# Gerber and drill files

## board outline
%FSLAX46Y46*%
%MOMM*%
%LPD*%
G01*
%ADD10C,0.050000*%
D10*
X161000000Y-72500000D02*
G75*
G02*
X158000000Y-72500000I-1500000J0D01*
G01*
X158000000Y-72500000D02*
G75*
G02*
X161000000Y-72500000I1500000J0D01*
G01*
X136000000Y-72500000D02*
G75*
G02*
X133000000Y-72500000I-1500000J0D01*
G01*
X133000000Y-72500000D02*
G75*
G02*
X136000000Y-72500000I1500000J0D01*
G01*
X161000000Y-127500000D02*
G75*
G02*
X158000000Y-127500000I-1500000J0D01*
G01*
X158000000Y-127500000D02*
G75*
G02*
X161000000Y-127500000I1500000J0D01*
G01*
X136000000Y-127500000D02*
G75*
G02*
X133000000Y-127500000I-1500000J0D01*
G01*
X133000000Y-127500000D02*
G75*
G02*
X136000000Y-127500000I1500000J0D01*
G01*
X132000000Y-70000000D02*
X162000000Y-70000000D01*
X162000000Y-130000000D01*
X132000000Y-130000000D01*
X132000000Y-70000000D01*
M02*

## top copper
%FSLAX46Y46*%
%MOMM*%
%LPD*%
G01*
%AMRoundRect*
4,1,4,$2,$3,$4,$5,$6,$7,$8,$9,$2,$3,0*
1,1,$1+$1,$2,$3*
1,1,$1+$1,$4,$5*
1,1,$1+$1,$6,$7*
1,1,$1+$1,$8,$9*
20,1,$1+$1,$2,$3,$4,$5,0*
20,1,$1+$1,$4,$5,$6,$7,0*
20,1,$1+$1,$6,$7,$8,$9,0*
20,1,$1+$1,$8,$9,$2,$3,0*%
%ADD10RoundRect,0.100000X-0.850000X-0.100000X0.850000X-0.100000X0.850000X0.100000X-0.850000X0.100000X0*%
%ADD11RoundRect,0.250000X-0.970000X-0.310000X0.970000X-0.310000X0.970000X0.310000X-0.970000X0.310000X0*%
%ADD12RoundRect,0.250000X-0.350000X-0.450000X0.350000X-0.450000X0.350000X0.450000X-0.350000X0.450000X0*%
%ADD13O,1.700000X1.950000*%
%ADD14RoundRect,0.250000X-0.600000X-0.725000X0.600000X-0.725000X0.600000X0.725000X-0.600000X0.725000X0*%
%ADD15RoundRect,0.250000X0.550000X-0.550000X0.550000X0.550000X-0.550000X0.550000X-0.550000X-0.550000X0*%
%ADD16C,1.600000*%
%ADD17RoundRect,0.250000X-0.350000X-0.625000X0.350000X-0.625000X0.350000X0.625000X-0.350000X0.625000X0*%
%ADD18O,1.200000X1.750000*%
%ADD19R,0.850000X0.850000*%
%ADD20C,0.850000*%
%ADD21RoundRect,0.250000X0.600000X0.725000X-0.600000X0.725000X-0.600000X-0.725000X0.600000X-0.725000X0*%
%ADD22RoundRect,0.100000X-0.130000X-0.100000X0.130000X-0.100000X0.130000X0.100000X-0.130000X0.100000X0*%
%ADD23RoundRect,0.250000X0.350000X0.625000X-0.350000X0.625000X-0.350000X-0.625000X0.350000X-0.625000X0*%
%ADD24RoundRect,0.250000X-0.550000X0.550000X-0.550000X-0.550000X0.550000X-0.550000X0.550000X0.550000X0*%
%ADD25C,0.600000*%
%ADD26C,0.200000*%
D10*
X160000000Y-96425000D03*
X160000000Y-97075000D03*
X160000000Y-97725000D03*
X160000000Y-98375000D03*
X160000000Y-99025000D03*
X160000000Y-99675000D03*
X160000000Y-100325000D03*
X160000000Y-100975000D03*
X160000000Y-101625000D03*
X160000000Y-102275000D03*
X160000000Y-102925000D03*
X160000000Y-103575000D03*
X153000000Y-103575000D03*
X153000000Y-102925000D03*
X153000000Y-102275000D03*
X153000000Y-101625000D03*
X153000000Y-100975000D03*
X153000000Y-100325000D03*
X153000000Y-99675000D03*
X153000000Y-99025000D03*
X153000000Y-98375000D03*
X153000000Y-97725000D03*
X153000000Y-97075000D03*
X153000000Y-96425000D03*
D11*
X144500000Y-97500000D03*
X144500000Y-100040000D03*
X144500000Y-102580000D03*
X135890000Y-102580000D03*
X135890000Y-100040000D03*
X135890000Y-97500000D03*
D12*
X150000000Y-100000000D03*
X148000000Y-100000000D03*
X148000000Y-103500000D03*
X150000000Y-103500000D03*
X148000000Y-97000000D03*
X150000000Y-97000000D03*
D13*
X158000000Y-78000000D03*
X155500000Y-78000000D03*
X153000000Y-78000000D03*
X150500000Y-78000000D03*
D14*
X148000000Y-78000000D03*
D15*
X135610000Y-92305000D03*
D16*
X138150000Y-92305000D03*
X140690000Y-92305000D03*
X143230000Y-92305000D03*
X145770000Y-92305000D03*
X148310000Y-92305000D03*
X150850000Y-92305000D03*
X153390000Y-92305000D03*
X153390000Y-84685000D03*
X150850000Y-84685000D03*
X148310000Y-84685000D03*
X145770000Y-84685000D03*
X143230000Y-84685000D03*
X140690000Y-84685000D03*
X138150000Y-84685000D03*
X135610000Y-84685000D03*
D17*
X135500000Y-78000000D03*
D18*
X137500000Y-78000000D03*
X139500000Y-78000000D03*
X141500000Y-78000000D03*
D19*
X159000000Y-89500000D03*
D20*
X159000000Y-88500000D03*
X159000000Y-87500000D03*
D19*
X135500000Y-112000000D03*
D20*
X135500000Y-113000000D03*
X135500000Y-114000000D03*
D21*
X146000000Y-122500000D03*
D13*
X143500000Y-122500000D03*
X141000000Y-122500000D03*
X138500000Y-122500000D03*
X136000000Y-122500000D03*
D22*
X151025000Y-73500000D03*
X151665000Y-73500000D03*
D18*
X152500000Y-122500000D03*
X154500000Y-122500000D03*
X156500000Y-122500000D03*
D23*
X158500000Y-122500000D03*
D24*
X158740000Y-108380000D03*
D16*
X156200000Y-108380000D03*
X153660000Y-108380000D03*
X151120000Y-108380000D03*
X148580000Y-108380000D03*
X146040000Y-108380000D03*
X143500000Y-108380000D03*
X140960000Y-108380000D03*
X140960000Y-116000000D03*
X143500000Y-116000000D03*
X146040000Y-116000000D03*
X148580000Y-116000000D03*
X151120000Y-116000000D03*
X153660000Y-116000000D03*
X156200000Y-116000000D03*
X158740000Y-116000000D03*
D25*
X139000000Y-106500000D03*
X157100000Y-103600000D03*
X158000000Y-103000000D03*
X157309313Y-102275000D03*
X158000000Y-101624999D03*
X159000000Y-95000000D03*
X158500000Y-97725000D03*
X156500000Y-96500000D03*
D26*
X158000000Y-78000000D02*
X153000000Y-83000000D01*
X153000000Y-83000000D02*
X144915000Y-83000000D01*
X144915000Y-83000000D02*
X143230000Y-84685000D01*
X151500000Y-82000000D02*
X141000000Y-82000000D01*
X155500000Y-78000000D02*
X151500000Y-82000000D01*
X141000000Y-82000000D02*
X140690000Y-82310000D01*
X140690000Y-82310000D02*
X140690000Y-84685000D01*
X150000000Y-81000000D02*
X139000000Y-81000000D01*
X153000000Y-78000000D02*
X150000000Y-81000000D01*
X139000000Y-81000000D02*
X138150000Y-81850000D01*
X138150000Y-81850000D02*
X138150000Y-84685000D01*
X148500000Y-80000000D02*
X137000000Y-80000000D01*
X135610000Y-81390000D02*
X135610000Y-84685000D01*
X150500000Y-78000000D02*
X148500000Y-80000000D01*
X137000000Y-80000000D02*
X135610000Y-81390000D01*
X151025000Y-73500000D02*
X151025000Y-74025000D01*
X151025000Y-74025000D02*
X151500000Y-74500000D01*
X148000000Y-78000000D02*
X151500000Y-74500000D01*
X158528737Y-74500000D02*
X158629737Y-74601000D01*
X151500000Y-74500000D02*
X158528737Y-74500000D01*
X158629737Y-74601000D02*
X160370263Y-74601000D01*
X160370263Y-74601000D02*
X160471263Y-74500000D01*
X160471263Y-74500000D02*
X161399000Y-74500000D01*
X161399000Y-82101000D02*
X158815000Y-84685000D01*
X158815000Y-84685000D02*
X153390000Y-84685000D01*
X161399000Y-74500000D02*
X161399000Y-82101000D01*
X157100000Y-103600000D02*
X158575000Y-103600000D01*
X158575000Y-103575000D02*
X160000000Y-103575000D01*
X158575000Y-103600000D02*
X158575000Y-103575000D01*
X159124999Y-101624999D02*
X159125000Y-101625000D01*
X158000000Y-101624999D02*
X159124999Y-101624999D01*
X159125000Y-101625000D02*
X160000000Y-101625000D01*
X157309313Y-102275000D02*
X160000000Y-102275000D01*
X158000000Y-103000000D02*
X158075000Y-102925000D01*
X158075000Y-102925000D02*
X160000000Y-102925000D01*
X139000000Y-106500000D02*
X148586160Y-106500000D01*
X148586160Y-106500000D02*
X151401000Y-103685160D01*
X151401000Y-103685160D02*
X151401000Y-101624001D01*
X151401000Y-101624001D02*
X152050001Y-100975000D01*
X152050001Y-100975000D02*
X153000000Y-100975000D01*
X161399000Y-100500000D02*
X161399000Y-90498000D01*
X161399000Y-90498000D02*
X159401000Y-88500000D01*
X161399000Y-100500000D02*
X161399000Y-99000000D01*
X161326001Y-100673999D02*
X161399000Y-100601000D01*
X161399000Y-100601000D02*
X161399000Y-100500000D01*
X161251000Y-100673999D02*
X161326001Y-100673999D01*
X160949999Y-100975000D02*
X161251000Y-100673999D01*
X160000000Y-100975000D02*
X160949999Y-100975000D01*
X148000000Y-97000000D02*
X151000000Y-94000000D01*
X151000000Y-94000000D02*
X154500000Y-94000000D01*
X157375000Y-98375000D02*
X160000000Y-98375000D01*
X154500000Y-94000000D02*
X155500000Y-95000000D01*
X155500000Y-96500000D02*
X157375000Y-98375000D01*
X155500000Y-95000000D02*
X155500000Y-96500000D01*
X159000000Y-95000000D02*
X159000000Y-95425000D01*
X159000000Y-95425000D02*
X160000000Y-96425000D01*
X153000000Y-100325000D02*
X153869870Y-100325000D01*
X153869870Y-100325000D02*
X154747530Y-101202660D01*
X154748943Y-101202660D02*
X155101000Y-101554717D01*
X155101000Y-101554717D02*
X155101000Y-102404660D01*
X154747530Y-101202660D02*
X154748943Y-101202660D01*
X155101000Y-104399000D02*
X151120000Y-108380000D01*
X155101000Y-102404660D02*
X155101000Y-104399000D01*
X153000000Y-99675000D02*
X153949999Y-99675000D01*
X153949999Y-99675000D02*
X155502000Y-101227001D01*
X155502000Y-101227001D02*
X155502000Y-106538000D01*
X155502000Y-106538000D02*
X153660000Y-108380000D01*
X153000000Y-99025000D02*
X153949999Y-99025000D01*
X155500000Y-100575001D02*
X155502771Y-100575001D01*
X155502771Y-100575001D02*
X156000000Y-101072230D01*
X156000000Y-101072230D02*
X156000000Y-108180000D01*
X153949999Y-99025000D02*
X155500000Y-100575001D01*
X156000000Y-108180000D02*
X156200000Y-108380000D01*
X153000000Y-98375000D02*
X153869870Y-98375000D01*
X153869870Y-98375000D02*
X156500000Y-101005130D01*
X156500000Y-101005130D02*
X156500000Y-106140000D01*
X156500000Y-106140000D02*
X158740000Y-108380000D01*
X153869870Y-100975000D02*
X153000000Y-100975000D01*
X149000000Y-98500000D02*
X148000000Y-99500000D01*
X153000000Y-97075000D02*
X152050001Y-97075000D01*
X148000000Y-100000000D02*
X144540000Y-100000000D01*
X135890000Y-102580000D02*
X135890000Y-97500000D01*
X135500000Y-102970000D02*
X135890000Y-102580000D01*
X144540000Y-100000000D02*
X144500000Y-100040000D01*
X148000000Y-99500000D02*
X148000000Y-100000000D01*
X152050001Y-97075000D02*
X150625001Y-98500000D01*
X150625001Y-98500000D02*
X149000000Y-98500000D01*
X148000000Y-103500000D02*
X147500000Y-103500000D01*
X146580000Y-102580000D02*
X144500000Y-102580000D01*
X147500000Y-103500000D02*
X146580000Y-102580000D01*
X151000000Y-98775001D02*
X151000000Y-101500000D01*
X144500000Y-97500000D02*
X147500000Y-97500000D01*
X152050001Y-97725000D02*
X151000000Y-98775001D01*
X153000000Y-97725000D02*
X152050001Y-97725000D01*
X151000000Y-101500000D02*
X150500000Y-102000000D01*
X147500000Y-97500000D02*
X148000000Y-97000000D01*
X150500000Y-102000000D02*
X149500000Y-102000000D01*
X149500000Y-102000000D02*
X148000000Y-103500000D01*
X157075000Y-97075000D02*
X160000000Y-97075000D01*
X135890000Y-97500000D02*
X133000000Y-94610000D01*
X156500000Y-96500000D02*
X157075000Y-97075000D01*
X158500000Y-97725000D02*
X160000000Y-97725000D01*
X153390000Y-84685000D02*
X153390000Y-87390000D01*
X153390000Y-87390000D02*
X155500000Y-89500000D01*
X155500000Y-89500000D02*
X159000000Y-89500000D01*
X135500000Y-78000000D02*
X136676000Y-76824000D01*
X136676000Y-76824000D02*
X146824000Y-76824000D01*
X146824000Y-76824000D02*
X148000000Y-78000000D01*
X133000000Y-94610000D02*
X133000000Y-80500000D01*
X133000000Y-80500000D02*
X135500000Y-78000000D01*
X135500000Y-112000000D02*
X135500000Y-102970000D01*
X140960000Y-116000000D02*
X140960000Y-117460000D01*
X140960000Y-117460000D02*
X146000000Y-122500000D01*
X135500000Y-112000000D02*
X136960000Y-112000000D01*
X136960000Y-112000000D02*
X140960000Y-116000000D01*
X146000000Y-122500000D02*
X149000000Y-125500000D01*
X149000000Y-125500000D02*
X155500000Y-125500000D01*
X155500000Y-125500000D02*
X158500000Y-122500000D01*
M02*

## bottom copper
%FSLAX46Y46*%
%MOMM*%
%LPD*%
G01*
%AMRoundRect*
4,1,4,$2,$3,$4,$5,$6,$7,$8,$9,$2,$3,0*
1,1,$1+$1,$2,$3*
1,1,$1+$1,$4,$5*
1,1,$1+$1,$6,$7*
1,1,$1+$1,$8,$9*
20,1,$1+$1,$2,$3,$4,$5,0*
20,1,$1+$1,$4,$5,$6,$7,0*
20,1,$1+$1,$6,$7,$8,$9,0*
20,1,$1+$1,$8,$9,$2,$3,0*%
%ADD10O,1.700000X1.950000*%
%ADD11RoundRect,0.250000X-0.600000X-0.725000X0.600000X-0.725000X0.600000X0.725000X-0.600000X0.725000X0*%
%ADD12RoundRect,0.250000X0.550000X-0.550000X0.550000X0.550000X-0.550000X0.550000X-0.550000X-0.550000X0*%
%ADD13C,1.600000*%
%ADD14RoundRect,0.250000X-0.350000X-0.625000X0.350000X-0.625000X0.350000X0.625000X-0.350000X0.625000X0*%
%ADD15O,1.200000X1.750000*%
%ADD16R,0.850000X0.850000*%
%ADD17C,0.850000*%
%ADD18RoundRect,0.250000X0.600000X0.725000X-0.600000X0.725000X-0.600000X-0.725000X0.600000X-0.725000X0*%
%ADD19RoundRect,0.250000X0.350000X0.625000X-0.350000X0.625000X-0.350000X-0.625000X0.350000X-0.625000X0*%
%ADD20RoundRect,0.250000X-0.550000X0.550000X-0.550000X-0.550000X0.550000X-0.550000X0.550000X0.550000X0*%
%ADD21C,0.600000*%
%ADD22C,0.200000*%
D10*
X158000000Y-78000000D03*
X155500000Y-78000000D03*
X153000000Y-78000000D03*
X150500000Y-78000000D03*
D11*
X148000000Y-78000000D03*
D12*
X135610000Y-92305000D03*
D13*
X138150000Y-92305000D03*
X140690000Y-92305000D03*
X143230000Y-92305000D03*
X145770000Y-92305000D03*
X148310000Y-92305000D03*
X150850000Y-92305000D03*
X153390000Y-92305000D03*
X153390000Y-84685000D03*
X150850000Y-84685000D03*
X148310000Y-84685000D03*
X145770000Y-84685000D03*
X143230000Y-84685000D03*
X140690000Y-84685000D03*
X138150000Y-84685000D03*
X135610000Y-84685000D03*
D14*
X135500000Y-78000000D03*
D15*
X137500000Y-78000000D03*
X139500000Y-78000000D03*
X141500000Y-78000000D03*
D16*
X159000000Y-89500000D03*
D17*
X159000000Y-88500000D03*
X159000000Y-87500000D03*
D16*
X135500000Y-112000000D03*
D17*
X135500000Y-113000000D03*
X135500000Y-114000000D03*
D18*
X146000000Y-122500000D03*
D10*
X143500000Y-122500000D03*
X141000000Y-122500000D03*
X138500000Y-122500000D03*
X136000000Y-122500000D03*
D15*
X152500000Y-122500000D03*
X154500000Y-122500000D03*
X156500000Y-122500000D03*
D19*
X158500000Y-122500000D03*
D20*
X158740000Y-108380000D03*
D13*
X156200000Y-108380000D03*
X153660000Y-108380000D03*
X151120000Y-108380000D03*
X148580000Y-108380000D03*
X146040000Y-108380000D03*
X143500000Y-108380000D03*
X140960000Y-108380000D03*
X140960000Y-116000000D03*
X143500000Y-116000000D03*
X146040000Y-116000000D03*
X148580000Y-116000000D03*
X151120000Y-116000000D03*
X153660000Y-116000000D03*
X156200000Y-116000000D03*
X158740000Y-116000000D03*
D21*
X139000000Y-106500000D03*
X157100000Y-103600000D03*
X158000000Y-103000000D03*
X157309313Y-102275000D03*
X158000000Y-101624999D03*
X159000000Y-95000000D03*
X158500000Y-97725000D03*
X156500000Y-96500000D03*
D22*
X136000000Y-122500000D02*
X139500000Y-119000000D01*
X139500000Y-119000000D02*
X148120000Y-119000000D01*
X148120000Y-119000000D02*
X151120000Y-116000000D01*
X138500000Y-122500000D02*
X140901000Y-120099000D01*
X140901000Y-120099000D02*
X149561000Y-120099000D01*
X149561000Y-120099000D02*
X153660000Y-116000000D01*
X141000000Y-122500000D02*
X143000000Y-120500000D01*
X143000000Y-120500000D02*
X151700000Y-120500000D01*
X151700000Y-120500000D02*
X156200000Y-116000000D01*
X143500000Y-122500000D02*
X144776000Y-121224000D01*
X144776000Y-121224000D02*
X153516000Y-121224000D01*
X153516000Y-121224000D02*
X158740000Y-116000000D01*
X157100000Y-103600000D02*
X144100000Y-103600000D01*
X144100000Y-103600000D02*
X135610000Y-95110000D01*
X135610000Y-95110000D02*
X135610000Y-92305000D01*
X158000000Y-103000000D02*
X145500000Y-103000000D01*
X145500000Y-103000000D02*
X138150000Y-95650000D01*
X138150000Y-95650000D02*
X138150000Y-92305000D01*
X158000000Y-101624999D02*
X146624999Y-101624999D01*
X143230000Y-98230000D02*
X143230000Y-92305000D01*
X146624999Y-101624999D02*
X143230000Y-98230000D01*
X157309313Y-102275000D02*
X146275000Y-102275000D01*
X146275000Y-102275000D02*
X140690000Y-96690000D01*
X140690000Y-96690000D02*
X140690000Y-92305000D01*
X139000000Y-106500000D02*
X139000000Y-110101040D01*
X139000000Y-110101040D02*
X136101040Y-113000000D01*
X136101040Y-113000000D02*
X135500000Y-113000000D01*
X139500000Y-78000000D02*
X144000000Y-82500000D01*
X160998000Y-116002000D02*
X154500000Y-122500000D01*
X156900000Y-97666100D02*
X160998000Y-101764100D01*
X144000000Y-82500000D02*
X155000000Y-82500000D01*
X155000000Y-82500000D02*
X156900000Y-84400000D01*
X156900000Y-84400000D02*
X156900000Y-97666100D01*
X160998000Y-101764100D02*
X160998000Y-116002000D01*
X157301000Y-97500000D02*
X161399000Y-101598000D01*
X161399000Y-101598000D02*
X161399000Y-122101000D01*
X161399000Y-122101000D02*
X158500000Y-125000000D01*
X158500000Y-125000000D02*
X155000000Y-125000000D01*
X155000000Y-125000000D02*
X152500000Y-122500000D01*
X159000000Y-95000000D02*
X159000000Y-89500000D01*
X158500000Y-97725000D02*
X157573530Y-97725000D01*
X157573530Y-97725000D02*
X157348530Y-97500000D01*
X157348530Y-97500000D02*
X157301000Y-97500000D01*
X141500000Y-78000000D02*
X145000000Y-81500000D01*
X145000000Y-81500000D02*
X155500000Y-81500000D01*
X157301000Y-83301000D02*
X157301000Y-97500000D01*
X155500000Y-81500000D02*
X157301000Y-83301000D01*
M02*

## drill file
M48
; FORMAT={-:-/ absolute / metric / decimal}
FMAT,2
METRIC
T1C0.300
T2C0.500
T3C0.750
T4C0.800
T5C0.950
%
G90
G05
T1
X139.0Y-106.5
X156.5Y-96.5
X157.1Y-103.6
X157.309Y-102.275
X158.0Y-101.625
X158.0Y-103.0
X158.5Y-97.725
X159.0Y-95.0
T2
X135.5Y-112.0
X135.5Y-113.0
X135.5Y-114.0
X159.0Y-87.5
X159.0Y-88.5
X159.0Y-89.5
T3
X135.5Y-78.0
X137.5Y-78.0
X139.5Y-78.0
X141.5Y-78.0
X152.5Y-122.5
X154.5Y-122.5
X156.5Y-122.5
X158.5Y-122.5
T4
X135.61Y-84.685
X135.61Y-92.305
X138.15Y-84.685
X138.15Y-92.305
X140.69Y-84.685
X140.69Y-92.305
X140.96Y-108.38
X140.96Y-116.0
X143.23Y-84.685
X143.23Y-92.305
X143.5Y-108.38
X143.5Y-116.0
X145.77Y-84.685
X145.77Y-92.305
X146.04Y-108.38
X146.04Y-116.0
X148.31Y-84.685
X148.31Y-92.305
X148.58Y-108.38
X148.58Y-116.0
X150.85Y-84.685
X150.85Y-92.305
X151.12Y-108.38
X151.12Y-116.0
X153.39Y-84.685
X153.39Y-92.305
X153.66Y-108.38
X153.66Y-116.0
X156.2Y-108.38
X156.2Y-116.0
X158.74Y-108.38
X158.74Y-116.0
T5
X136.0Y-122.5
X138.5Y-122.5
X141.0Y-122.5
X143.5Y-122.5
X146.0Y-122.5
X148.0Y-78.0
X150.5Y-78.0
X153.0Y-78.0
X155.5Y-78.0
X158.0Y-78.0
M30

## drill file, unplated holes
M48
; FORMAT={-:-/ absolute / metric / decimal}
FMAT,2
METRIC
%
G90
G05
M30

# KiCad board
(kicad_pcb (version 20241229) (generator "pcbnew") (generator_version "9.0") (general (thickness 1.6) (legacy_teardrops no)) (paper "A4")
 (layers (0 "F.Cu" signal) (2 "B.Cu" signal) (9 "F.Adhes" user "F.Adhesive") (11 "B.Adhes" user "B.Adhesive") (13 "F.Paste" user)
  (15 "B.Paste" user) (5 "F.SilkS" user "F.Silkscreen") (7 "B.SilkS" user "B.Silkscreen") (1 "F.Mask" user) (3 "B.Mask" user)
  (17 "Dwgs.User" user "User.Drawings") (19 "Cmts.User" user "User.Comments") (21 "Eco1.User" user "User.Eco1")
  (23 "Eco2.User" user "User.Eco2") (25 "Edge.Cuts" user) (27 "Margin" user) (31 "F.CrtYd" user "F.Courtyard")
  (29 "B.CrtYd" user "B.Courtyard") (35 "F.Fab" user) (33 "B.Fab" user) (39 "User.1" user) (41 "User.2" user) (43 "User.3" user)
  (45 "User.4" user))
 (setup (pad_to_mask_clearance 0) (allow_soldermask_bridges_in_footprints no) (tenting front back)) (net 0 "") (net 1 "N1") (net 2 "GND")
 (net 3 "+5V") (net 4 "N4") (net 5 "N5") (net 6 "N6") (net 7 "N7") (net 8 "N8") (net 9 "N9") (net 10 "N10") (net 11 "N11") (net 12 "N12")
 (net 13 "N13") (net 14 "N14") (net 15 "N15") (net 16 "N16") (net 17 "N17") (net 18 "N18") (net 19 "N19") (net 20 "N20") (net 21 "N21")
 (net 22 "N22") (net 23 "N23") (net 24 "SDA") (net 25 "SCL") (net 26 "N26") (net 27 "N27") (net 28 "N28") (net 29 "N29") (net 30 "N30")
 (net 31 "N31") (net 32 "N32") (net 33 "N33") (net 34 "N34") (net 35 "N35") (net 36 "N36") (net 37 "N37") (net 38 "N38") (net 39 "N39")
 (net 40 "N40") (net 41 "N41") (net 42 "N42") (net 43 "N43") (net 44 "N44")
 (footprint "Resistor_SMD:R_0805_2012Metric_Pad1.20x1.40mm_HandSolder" (layer "F.Cu") (at 149 103.5)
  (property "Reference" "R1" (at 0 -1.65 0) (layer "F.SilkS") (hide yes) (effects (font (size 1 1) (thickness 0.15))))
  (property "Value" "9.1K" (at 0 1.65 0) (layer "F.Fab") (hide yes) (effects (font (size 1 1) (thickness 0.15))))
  (pad "1" smd roundrect (at -1 0) (size 1.2 1.4) (layers "F.Cu" "F.Mask" "F.Paste") (roundrect_rratio 0.208333) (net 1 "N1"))
  (pad "2" smd roundrect (at 1 0) (size 1.2 1.4) (layers "F.Cu" "F.Mask" "F.Paste") (roundrect_rratio 0.208333) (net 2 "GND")))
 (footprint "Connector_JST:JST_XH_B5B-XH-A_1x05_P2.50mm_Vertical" (layer "F.Cu") (at 148 78)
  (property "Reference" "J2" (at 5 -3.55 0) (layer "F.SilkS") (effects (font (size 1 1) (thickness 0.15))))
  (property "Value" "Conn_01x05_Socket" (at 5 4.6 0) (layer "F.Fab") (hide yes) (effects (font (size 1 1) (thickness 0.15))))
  (pad "1" thru_hole roundrect (at 0 0) (size 1.7 1.95) (drill 0.95) (layers "*.Cu" "*.Mask") (remove_unused_layers no)
   (roundrect_rratio 0.147059) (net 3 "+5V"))
  (pad "2" thru_hole oval (at 2.5 0) (size 1.7 1.95) (drill 0.95) (layers "*.Cu" "*.Mask") (remove_unused_layers no) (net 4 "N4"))
  (pad "3" thru_hole oval (at 5 0) (size 1.7 1.95) (drill 0.95) (layers "*.Cu" "*.Mask") (remove_unused_layers no) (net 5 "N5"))
  (pad "4" thru_hole oval (at 7.5 0) (size 1.7 1.95) (drill 0.95) (layers "*.Cu" "*.Mask") (remove_unused_layers no) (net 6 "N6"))
  (pad "5" thru_hole oval (at 10 0) (size 1.7 1.95) (drill 0.95) (layers "*.Cu" "*.Mask") (remove_unused_layers no) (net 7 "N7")))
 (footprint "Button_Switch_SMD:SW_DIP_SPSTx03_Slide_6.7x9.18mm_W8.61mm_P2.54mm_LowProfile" (layer "F.Cu") (at 140.195 100.04)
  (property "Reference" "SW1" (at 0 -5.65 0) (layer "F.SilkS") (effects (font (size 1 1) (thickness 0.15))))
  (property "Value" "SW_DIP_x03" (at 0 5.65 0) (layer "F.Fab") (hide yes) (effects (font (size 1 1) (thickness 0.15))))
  (pad "1" smd roundrect (at -4.305 -2.54) (size 2.44 1.12) (layers "F.Cu" "F.Mask" "F.Paste") (roundrect_rratio 0.223214) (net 3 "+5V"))
  (pad "2" smd roundrect (at -4.305 0) (size 2.44 1.12) (layers "F.Cu" "F.Mask" "F.Paste") (roundrect_rratio 0.223214) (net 3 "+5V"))
  (pad "3" smd roundrect (at -4.305 2.54) (size 2.44 1.12) (layers "F.Cu" "F.Mask" "F.Paste") (roundrect_rratio 0.223214) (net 3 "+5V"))
  (pad "4" smd roundrect (at 4.305 2.54) (size 2.44 1.12) (layers "F.Cu" "F.Mask" "F.Paste") (roundrect_rratio 0.223214) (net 1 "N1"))
  (pad "5" smd roundrect (at 4.305 0) (size 2.44 1.12) (layers "F.Cu" "F.Mask" "F.Paste") (roundrect_rratio 0.223214) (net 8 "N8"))
  (pad "6" smd roundrect (at 4.305 -2.54) (size 2.44 1.12) (layers "F.Cu" "F.Mask" "F.Paste") (roundrect_rratio 0.223214) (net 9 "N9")))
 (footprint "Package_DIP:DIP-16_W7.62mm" (layer "F.Cu") (at 158.74 108.38 -90)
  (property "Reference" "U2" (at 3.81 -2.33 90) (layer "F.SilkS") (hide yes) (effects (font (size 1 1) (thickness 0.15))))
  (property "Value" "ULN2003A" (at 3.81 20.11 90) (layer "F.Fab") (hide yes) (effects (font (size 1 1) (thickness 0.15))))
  (pad "1" thru_hole roundrect (at 0 0 270) (size 1.6 1.6) (drill 0.8) (layers "*.Cu" "*.Mask") (remove_unused_layers no)
   (roundrect_rratio 0.15625) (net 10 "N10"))
  (pad "2" thru_hole circle (at 0 2.54 270) (size 1.6 1.6) (drill 0.8) (layers "*.Cu" "*.Mask") (remove_unused_layers no) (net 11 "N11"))
  (pad "3" thru_hole circle (at 0 5.08 270) (size 1.6 1.6) (drill 0.8) (layers "*.Cu" "*.Mask") (remove_unused_layers no) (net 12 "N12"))
  (pad "4" thru_hole circle (at 0 7.62 270) (size 1.6 1.6) (drill 0.8) (layers "*.Cu" "*.Mask") (remove_unused_layers no) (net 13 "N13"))
  (pad "5" thru_hole circle (at 0 10.16 270) (size 1.6 1.6) (drill 0.8) (layers "*.Cu" "*.Mask") (remove_unused_layers no) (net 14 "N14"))
  (pad "6" thru_hole circle (at 0 12.7 270) (size 1.6 1.6) (drill 0.8) (layers "*.Cu" "*.Mask") (remove_unused_layers no) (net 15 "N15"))
  (pad "7" thru_hole circle (at 0 15.24 270) (size 1.6 1.6) (drill 0.8) (layers "*.Cu" "*.Mask") (remove_unused_layers no) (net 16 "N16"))
  (pad "8" thru_hole circle (at 0 17.78 270) (size 1.6 1.6) (drill 0.8) (layers "*.Cu" "*.Mask") (remove_unused_layers no) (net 2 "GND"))
  (pad "9" thru_hole circle (at 7.62 17.78 270) (size 1.6 1.6) (drill 0.8) (layers "*.Cu" "*.Mask") (remove_unused_layers no) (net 3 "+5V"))
  (pad "10" thru_hole circle (at 7.62 15.24 270) (size 1.6 1.6) (drill 0.8) (layers "*.Cu" "*.Mask") (remove_unused_layers no)
   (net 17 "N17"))
  (pad "11" thru_hole circle (at 7.62 12.7 270) (size 1.6 1.6) (drill 0.8) (layers "*.Cu" "*.Mask") (remove_unused_layers no) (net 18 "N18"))
  (pad "12" thru_hole circle (at 7.62 10.16 270) (size 1.6 1.6) (drill 0.8) (layers "*.Cu" "*.Mask") (remove_unused_layers no)
   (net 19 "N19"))
  (pad "13" thru_hole circle (at 7.62 7.62 270) (size 1.6 1.6) (drill 0.8) (layers "*.Cu" "*.Mask") (remove_unused_layers no) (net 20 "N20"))
  (pad "14" thru_hole circle (at 7.62 5.08 270) (size 1.6 1.6) (drill 0.8) (layers "*.Cu" "*.Mask") (remove_unused_layers no) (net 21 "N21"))
  (pad "15" thru_hole circle (at 7.62 2.54 270) (size 1.6 1.6) (drill 0.8) (layers "*.Cu" "*.Mask") (remove_unused_layers no) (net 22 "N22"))
  (pad "16" thru_hole circle (at 7.62 0 270) (size 1.6 1.6) (drill 0.8) (layers "*.Cu" "*.Mask") (remove_unused_layers no) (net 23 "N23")))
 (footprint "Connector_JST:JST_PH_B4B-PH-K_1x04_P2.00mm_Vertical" (layer "F.Cu") (at 158.5 122.5 180)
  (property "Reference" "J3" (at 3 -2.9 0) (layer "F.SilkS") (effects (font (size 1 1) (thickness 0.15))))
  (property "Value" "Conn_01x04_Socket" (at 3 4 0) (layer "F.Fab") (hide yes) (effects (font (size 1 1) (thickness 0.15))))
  (pad "1" thru_hole roundrect (at 0 0 180) (size 1.2 1.75) (drill 0.75) (layers "*.Cu" "*.Mask") (remove_unused_layers no)
   (roundrect_rratio 0.208333) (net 3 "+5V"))
  (pad "2" thru_hole oval (at 2 0 180) (size 1.2 1.75) (drill 0.75) (layers "*.Cu" "*.Mask") (remove_unused_layers no) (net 2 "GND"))
  (pad "3" thru_hole oval (at 4 0 180) (size 1.2 1.75) (drill 0.75) (layers "*.Cu" "*.Mask") (remove_unused_layers no) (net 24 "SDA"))
  (pad "4" thru_hole oval (at 6 0 180) (size 1.2 1.75) (drill 0.75) (layers "*.Cu" "*.Mask") (remove_unused_layers no) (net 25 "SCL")))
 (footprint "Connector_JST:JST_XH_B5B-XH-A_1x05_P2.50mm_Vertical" (layer "F.Cu") (at 146 122.5 180)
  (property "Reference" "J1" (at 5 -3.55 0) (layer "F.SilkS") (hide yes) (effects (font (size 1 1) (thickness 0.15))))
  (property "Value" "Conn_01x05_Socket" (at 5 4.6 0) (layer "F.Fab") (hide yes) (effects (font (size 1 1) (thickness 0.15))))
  (pad "1" thru_hole roundrect (at 0 0 180) (size 1.7 1.95) (drill 0.95) (layers "*.Cu" "*.Mask") (remove_unused_layers no)
   (roundrect_rratio 0.147059) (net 3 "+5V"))
  (pad "2" thru_hole oval (at 2.5 0 180) (size 1.7 1.95) (drill 0.95) (layers "*.Cu" "*.Mask") (remove_unused_layers no) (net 23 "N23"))
  (pad "3" thru_hole oval (at 5 0 180) (size 1.7 1.95) (drill 0.95) (layers "*.Cu" "*.Mask") (remove_unused_layers no) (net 22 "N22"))
  (pad "4" thru_hole oval (at 7.5 0 180) (size 1.7 1.95) (drill 0.95) (layers "*.Cu" "*.Mask") (remove_unused_layers no) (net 21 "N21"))
  (pad "5" thru_hole oval (at 10 0 180) (size 1.7 1.95) (drill 0.95) (layers "*.Cu" "*.Mask") (remove_unused_layers no) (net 20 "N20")))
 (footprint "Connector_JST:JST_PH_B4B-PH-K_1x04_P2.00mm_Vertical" (layer "F.Cu") (at 135.5 78)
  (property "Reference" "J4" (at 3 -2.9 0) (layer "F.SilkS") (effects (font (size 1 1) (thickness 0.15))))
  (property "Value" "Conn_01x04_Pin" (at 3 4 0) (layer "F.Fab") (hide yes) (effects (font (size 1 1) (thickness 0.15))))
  (pad "1" thru_hole roundrect (at 0 0) (size 1.2 1.75) (drill 0.75) (layers "*.Cu" "*.Mask") (remove_unused_layers no)
   (roundrect_rratio 0.208333) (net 3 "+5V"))
  (pad "2" thru_hole oval (at 2 0) (size 1.2 1.75) (drill 0.75) (layers "*.Cu" "*.Mask") (remove_unused_layers no) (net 2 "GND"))
  (pad "3" thru_hole oval (at 4 0) (size 1.2 1.75) (drill 0.75) (layers "*.Cu" "*.Mask") (remove_unused_layers no) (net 24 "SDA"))
  (pad "4" thru_hole oval (at 6 0) (size 1.2 1.75) (drill 0.75) (layers "*.Cu" "*.Mask") (remove_unused_layers no) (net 25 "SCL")))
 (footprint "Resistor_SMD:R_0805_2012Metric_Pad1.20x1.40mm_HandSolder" (layer "F.Cu") (at 149 100)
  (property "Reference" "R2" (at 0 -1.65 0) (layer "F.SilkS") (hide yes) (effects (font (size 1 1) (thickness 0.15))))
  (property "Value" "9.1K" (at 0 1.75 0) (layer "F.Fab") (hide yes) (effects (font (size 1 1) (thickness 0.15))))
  (pad "1" smd roundrect (at -1 0) (size 1.2 1.4) (layers "F.Cu" "F.Mask" "F.Paste") (roundrect_rratio 0.208333) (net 8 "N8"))
  (pad "2" smd roundrect (at 1 0) (size 1.2 1.4) (layers "F.Cu" "F.Mask" "F.Paste") (roundrect_rratio 0.208333) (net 2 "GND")))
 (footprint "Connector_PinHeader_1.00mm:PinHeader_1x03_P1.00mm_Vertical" (layer "F.Cu") (at 159 89.5 180)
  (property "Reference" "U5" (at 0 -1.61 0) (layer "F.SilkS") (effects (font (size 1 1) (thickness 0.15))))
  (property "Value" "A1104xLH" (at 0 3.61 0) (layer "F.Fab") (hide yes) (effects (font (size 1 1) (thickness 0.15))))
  (pad "1" thru_hole rect (at 0 0 180) (size 0.85 0.85) (drill 0.5) (layers "*.Cu" "*.Mask") (remove_unused_layers no) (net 3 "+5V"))
  (pad "2" thru_hole circle (at 0 1 180) (size 0.85 0.85) (drill 0.5) (layers "*.Cu" "*.Mask") (remove_unused_layers no) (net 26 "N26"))
  (pad "3" thru_hole circle (at 0 2 180) (size 0.85 0.85) (drill 0.5) (layers "*.Cu" "*.Mask") (remove_unused_layers no) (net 2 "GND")))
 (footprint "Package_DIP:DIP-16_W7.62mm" (layer "F.Cu") (at 135.61 92.305 90)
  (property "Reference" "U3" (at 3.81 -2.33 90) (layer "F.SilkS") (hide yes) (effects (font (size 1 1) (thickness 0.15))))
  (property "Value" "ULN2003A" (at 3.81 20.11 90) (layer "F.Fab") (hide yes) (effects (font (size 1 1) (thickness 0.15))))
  (pad "1" thru_hole roundrect (at 0 0 90) (size 1.6 1.6) (drill 0.8) (layers "*.Cu" "*.Mask") (remove_unused_layers no)
   (roundrect_rratio 0.15625) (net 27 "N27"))
  (pad "2" thru_hole circle (at 0 2.54 90) (size 1.6 1.6) (drill 0.8) (layers "*.Cu" "*.Mask") (remove_unused_layers no) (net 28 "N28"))
  (pad "3" thru_hole circle (at 0 5.08 90) (size 1.6 1.6) (drill 0.8) (layers "*.Cu" "*.Mask") (remove_unused_layers no) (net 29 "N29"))
  (pad "4" thru_hole circle (at 0 7.62 90) (size 1.6 1.6) (drill 0.8) (layers "*.Cu" "*.Mask") (remove_unused_layers no) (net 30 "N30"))
  (pad "5" thru_hole circle (at 0 10.16 90) (size 1.6 1.6) (drill 0.8) (layers "*.Cu" "*.Mask") (remove_unused_layers no) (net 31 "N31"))
  (pad "6" thru_hole circle (at 0 12.7 90) (size 1.6 1.6) (drill 0.8) (layers "*.Cu" "*.Mask") (remove_unused_layers no) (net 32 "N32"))
  (pad "7" thru_hole circle (at 0 15.24 90) (size 1.6 1.6) (drill 0.8) (layers "*.Cu" "*.Mask") (remove_unused_layers no) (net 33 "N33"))
  (pad "8" thru_hole circle (at 0 17.78 90) (size 1.6 1.6) (drill 0.8) (layers "*.Cu" "*.Mask") (remove_unused_layers no) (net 2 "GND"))
  (pad "9" thru_hole circle (at 7.62 17.78 90) (size 1.6 1.6) (drill 0.8) (layers "*.Cu" "*.Mask") (remove_unused_layers no) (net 3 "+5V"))
  (pad "10" thru_hole circle (at 7.62 15.24 90) (size 1.6 1.6) (drill 0.8) (layers "*.Cu" "*.Mask") (remove_unused_layers no) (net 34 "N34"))
  (pad "11" thru_hole circle (at 7.62 12.7 90) (size 1.6 1.6) (drill 0.8) (layers "*.Cu" "*.Mask") (remove_unused_layers no) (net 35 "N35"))
  (pad "12" thru_hole circle (at 7.62 10.16 90) (size 1.6 1.6) (drill 0.8) (layers "*.Cu" "*.Mask") (remove_unused_layers no) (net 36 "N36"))
  (pad "13" thru_hole circle (at 7.62 7.62 90) (size 1.6 1.6) (drill 0.8) (layers "*.Cu" "*.Mask") (remove_unused_layers no) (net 7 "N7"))
  (pad "14" thru_hole circle (at 7.62 5.08 90) (size 1.6 1.6) (drill 0.8) (layers "*.Cu" "*.Mask") (remove_unused_layers no) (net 6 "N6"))
  (pad "15" thru_hole circle (at 7.62 2.54 90) (size 1.6 1.6) (drill 0.8) (layers "*.Cu" "*.Mask") (remove_unused_layers no) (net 5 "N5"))
  (pad "16" thru_hole circle (at 7.62 0 90) (size 1.6 1.6) (drill 0.8) (layers "*.Cu" "*.Mask") (remove_unused_layers no) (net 4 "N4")))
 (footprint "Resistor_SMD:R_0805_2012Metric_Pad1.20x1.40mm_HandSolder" (layer "F.Cu") (at 149 97)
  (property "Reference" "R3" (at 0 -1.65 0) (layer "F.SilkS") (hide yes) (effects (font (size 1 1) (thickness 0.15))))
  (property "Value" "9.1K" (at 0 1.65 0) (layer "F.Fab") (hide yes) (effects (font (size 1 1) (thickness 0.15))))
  (pad "1" smd roundrect (at -1 0) (size 1.2 1.4) (layers "F.Cu" "F.Mask" "F.Paste") (roundrect_rratio 0.208333) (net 9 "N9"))
  (pad "2" smd roundrect (at 1 0) (size 1.2 1.4) (layers "F.Cu" "F.Mask" "F.Paste") (roundrect_rratio 0.208333) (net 2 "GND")))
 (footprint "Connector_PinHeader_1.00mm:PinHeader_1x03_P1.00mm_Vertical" (layer "F.Cu") (at 135.5 112)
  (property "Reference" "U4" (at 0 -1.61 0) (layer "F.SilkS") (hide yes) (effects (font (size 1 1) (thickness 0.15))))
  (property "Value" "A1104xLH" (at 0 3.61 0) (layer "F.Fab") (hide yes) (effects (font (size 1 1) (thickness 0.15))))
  (pad "1" thru_hole rect (at 0 0) (size 0.85 0.85) (drill 0.5) (layers "*.Cu" "*.Mask") (remove_unused_layers no) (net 3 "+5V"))
  (pad "2" thru_hole circle (at 0 1) (size 0.85 0.85) (drill 0.5) (layers "*.Cu" "*.Mask") (remove_unused_layers no) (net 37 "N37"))
  (pad "3" thru_hole circle (at 0 2) (size 0.85 0.85) (drill 0.5) (layers "*.Cu" "*.Mask") (remove_unused_layers no) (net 2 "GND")))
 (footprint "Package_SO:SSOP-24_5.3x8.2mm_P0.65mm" (layer "F.Cu") (at 156.5 100)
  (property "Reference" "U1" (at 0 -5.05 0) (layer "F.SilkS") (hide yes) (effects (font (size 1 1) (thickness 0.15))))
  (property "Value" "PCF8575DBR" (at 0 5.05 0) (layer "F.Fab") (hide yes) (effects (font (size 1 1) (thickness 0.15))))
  (pad "1" smd roundrect (at -3.5 -3.575) (size 1.9 0.4) (layers "F.Cu" "F.Mask" "F.Paste") (roundrect_rratio 0.25) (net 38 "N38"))
  (pad "2" smd roundrect (at -3.5 -2.925) (size 1.9 0.4) (layers "F.Cu" "F.Mask" "F.Paste") (roundrect_rratio 0.25) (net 8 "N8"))
  (pad "3" smd roundrect (at -3.5 -2.275) (size 1.9 0.4) (layers "F.Cu" "F.Mask" "F.Paste") (roundrect_rratio 0.25) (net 1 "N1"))
  (pad "4" smd roundrect (at -3.5 -1.625) (size 1.9 0.4) (layers "F.Cu" "F.Mask" "F.Paste") (roundrect_rratio 0.25) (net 10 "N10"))
  (pad "5" smd roundrect (at -3.5 -0.975) (size 1.9 0.4) (layers "F.Cu" "F.Mask" "F.Paste") (roundrect_rratio 0.25) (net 11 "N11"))
  (pad "6" smd roundrect (at -3.5 -0.325) (size 1.9 0.4) (layers "F.Cu" "F.Mask" "F.Paste") (roundrect_rratio 0.25) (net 12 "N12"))
  (pad "7" smd roundrect (at -3.5 0.325) (size 1.9 0.4) (layers "F.Cu" "F.Mask" "F.Paste") (roundrect_rratio 0.25) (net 13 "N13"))
  (pad "8" smd roundrect (at -3.5 0.975) (size 1.9 0.4) (layers "F.Cu" "F.Mask" "F.Paste") (roundrect_rratio 0.25) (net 37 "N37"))
  (pad "9" smd roundrect (at -3.5 1.625) (size 1.9 0.4) (layers "F.Cu" "F.Mask" "F.Paste") (roundrect_rratio 0.25) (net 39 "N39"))
  (pad "10" smd roundrect (at -3.5 2.275) (size 1.9 0.4) (layers "F.Cu" "F.Mask" "F.Paste") (roundrect_rratio 0.25) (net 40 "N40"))
  (pad "11" smd roundrect (at -3.5 2.925) (size 1.9 0.4) (layers "F.Cu" "F.Mask" "F.Paste") (roundrect_rratio 0.25) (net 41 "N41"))
  (pad "12" smd roundrect (at -3.5 3.575) (size 1.9 0.4) (layers "F.Cu" "F.Mask" "F.Paste") (roundrect_rratio 0.25) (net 2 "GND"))
  (pad "13" smd roundrect (at 3.5 3.575) (size 1.9 0.4) (layers "F.Cu" "F.Mask" "F.Paste") (roundrect_rratio 0.25) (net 27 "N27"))
  (pad "14" smd roundrect (at 3.5 2.925) (size 1.9 0.4) (layers "F.Cu" "F.Mask" "F.Paste") (roundrect_rratio 0.25) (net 28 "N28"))
  (pad "15" smd roundrect (at 3.5 2.275) (size 1.9 0.4) (layers "F.Cu" "F.Mask" "F.Paste") (roundrect_rratio 0.25) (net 29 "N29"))
  (pad "16" smd roundrect (at 3.5 1.625) (size 1.9 0.4) (layers "F.Cu" "F.Mask" "F.Paste") (roundrect_rratio 0.25) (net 30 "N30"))
  (pad "17" smd roundrect (at 3.5 0.975) (size 1.9 0.4) (layers "F.Cu" "F.Mask" "F.Paste") (roundrect_rratio 0.25) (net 26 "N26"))
  (pad "18" smd roundrect (at 3.5 0.325) (size 1.9 0.4) (layers "F.Cu" "F.Mask" "F.Paste") (roundrect_rratio 0.25) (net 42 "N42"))
  (pad "19" smd roundrect (at 3.5 -0.325) (size 1.9 0.4) (layers "F.Cu" "F.Mask" "F.Paste") (roundrect_rratio 0.25) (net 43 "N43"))
  (pad "20" smd roundrect (at 3.5 -0.975) (size 1.9 0.4) (layers "F.Cu" "F.Mask" "F.Paste") (roundrect_rratio 0.25) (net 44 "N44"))
  (pad "21" smd roundrect (at 3.5 -1.625) (size 1.9 0.4) (layers "F.Cu" "F.Mask" "F.Paste") (roundrect_rratio 0.25) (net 9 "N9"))
  (pad "22" smd roundrect (at 3.5 -2.275) (size 1.9 0.4) (layers "F.Cu" "F.Mask" "F.Paste") (roundrect_rratio 0.25) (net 25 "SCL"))
  (pad "23" smd roundrect (at 3.5 -2.925) (size 1.9 0.4) (layers "F.Cu" "F.Mask" "F.Paste") (roundrect_rratio 0.25) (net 24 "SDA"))
  (pad "24" smd roundrect (at 3.5 -3.575) (size 1.9 0.4) (layers "F.Cu" "F.Mask" "F.Paste") (roundrect_rratio 0.25) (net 3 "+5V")))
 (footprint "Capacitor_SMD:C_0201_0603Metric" (layer "F.Cu") (at 151.345 73.5)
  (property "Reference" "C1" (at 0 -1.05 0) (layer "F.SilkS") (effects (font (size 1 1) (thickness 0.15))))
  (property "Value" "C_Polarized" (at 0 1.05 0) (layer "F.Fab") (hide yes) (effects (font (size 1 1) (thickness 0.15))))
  (pad "" smd roundrect (at -0.345 0) (size 0.318 0.36) (layers "F.Paste") (roundrect_rratio 0.25))
  (pad "" smd roundrect (at 0.345 0) (size 0.318 0.36) (layers "F.Paste") (roundrect_rratio 0.25))
  (pad "1" smd roundrect (at -0.32 0) (size 0.46 0.4) (layers "F.Cu" "F.Mask") (roundrect_rratio 0.25) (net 3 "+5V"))
  (pad "2" smd roundrect (at 0.32 0) (size 0.46 0.4) (layers "F.Cu" "F.Mask") (roundrect_rratio 0.25) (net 2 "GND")))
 (gr_circle (center 159.5 72.5) (end 161 72.5) (stroke (width 0.05) (type default)) (fill no) (layer "Edge.Cuts"))
 (gr_circle (center 134.5 72.5) (end 136 72.5) (stroke (width 0.05) (type default)) (fill no) (layer "Edge.Cuts"))
 (gr_circle (center 159.5 127.5) (end 161 127.5) (stroke (width 0.05) (type default)) (fill no) (layer "Edge.Cuts"))
 (gr_circle (center 134.5 127.5) (end 136 127.5) (stroke (width 0.05) (type default)) (fill no) (layer "Edge.Cuts"))
 (gr_rect (start 132 70) (end 162 130) (stroke (width 0.05) (type solid)) (fill no) (layer "Edge.Cuts"))
 (segment (start 155.5 89.5) (end 159 89.5) (width 0.2) (layer "F.Cu") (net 3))
 (segment (start 136.96 112) (end 140.96 116) (width 0.2) (layer "F.Cu") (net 3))
 (segment (start 159 95) (end 159 95.425) (width 0.2) (layer "F.Cu") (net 3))
 (segment (start 140.96 116) (end 140.96 117.46) (width 0.2) (layer "F.Cu") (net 3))
 (segment (start 149 125.5) (end 155.5 125.5) (width 0.2) (layer "F.Cu") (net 3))
 (segment (start 135.89 102.58) (end 135.89 97.5) (width 0.2) (layer "F.Cu") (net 3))
 (segment (start 151.025 73.5) (end 151.025 74.025) (width 0.2) (layer "F.Cu") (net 3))
 (segment (start 158.629737 74.601) (end 160.370263 74.601) (width 0.2) (layer "F.Cu") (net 3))
 (segment (start 153.39 87.39) (end 155.5 89.5) (width 0.2) (layer "F.Cu") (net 3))
 (segment (start 146 122.5) (end 149 125.5) (width 0.2) (layer "F.Cu") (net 3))
 (segment (start 135.5 78) (end 136.676 76.824) (width 0.2) (layer "F.Cu") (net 3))
 (segment (start 160.471263 74.5) (end 161.399 74.5) (width 0.2) (layer "F.Cu") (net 3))
 (segment (start 135.5 112) (end 136.96 112) (width 0.2) (layer "F.Cu") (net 3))
 (segment (start 151.025 74.025) (end 151.5 74.5) (width 0.2) (layer "F.Cu") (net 3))
 (segment (start 161.399 82.101) (end 158.815 84.685) (width 0.2) (layer "F.Cu") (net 3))
 (segment (start 161.399 74.5) (end 161.399 82.101) (width 0.2) (layer "F.Cu") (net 3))
 (segment (start 153.39 84.685) (end 153.39 87.39) (width 0.2) (layer "F.Cu") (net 3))
 (segment (start 135.5 102.97) (end 135.89 102.58) (width 0.2) (layer "F.Cu") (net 3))
 (segment (start 140.96 117.46) (end 146 122.5) (width 0.2) (layer "F.Cu") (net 3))
 (segment (start 158.528737 74.5) (end 158.629737 74.601) (width 0.2) (layer "F.Cu") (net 3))
 (segment (start 159 95.425) (end 160 96.425) (width 0.2) (layer "F.Cu") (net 3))
 (segment (start 135.5 112) (end 135.5 102.97) (width 0.2) (layer "F.Cu") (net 3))
 (segment (start 160.370263 74.601) (end 160.471263 74.5) (width 0.2) (layer "F.Cu") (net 3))
 (segment (start 135.89 97.5) (end 133 94.61) (width 0.2) (layer "F.Cu") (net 3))
 (segment (start 133 80.5) (end 135.5 78) (width 0.2) (layer "F.Cu") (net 3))
 (segment (start 148 78) (end 151.5 74.5) (width 0.2) (layer "F.Cu") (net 3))
 (segment (start 155.5 125.5) (end 158.5 122.5) (width 0.2) (layer "F.Cu") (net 3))
 (segment (start 133 94.61) (end 133 80.5) (width 0.2) (layer "F.Cu") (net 3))
 (segment (start 158.815 84.685) (end 153.39 84.685) (width 0.2) (layer "F.Cu") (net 3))
 (segment (start 146.824 76.824) (end 148 78) (width 0.2) (layer "F.Cu") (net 3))
 (segment (start 136.676 76.824) (end 146.824 76.824) (width 0.2) (layer "F.Cu") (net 3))
 (segment (start 151.5 74.5) (end 158.528737 74.5) (width 0.2) (layer "F.Cu") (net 3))
 (via (at 159 95) (size 0.6) (drill 0.3) (layers "F.Cu" "B.Cu") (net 3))
 (segment (start 159 95) (end 159 89.5) (width 0.2) (layer "B.Cu") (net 3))
 (segment (start 149.561 120.099) (end 153.66 116) (width 0.2) (layer "B.Cu") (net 21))
 (segment (start 138.5 122.5) (end 140.901 120.099) (width 0.2) (layer "B.Cu") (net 21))
 (segment (start 140.901 120.099) (end 149.561 120.099) (width 0.2) (layer "B.Cu") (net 21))
 (segment (start 144.776 121.224) (end 153.516 121.224) (width 0.2) (layer "B.Cu") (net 23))
 (segment (start 153.516 121.224) (end 158.74 116) (width 0.2) (layer "B.Cu") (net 23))
 (segment (start 143.5 122.5) (end 144.776 121.224) (width 0.2) (layer "B.Cu") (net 23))
 (segment (start 148.12 119) (end 151.12 116) (width 0.2) (layer "B.Cu") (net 20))
 (segment (start 136 122.5) (end 139.5 119) (width 0.2) (layer "B.Cu") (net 20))
 (segment (start 139.5 119) (end 148.12 119) (width 0.2) (layer "B.Cu") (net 20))
 (segment (start 143 120.5) (end 151.7 120.5) (width 0.2) (layer "B.Cu") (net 22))
 (segment (start 141 122.5) (end 143 120.5) (width 0.2) (layer "B.Cu") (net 22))
 (segment (start 151.7 120.5) (end 156.2 116) (width 0.2) (layer "B.Cu") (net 22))
 (segment (start 150.5 78) (end 148.5 80) (width 0.2) (layer "F.Cu") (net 4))
 (segment (start 135.61 81.39) (end 135.61 84.685) (width 0.2) (layer "F.Cu") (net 4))
 (segment (start 137 80) (end 135.61 81.39) (width 0.2) (layer "F.Cu") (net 4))
 (segment (start 148.5 80) (end 137 80) (width 0.2) (layer "F.Cu") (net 4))
 (segment (start 144.915 83) (end 143.23 84.685) (width 0.2) (layer "F.Cu") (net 7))
 (segment (start 153 83) (end 144.915 83) (width 0.2) (layer "F.Cu") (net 7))
 (segment (start 158 78) (end 153 83) (width 0.2) (layer "F.Cu") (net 7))
 (segment (start 150 81) (end 139 81) (width 0.2) (layer "F.Cu") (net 5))
 (segment (start 153 78) (end 150 81) (width 0.2) (layer "F.Cu") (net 5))
 (segment (start 139 81) (end 138.15 81.85) (width 0.2) (layer "F.Cu") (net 5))
 (segment (start 138.15 81.85) (end 138.15 84.685) (width 0.2) (layer "F.Cu") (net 5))
 (segment (start 151.5 82) (end 141 82) (width 0.2) (layer "F.Cu") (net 6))
 (segment (start 155.5 78) (end 151.5 82) (width 0.2) (layer "F.Cu") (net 6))
 (segment (start 140.69 82.31) (end 140.69 84.685) (width 0.2) (layer "F.Cu") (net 6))
 (segment (start 141 82) (end 140.69 82.31) (width 0.2) (layer "F.Cu") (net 6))
 (segment (start 149.5 102) (end 148 103.5) (width 0.2) (layer "F.Cu") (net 1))
 (segment (start 147.5 103.5) (end 146.58 102.58) (width 0.2) (layer "F.Cu") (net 1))
 (segment (start 153 97.725) (end 152.050001 97.725) (width 0.2) (layer "F.Cu") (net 1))
 (segment (start 150.5 102) (end 149.5 102) (width 0.2) (layer "F.Cu") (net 1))
 (segment (start 148 103.5) (end 147.5 103.5) (width 0.2) (layer "F.Cu") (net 1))
 (segment (start 146.58 102.58) (end 144.5 102.58) (width 0.2) (layer "F.Cu") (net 1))
 (segment (start 151 101.5) (end 150.5 102) (width 0.2) (layer "F.Cu") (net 1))
 (segment (start 152.050001 97.725) (end 151 98.775001) (width 0.2) (layer "F.Cu") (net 1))
 (segment (start 151 98.775001) (end 151 101.5) (width 0.2) (layer "F.Cu") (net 1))
 (segment (start 149 98.5) (end 148 99.5) (width 0.2) (layer "F.Cu") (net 8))
 (segment (start 148 99.5) (end 148 100) (width 0.2) (layer "F.Cu") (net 8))
 (segment (start 144.54 100) (end 144.5 100.04) (width 0.2) (layer "F.Cu") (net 8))
 (segment (start 150.625001 98.5) (end 149 98.5) (width 0.2) (layer "F.Cu") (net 8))
 (segment (start 148 100) (end 144.54 100) (width 0.2) (layer "F.Cu") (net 8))
 (segment (start 153 97.075) (end 152.050001 97.075) (width 0.2) (layer "F.Cu") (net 8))
 (segment (start 152.050001 97.075) (end 150.625001 98.5) (width 0.2) (layer "F.Cu") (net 8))
 (segment (start 154.5 94) (end 155.5 95) (width 0.2) (layer "F.Cu") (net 9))
 (segment (start 155.5 96.5) (end 157.375 98.375) (width 0.2) (layer "F.Cu") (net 9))
 (segment (start 147.5 97.5) (end 148 97) (width 0.2) (layer "F.Cu") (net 9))
 (segment (start 157.375 98.375) (end 160 98.375) (width 0.2) (layer "F.Cu") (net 9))
 (segment (start 144.5 97.5) (end 147.5 97.5) (width 0.2) (layer "F.Cu") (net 9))
 (segment (start 148 97) (end 151 94) (width 0.2) (layer "F.Cu") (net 9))
 (segment (start 151 94) (end 154.5 94) (width 0.2) (layer "F.Cu") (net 9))
 (segment (start 155.5 95) (end 155.5 96.5) (width 0.2) (layer "F.Cu") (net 9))
 (segment (start 159.124999 101.624999) (end 159.125 101.625) (width 0.2) (layer "F.Cu") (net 30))
 (segment (start 159.125 101.625) (end 160 101.625) (width 0.2) (layer "F.Cu") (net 30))
 (segment (start 158 101.624999) (end 159.124999 101.624999) (width 0.2) (layer "F.Cu") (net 30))
 (via (at 158 101.624999) (size 0.6) (drill 0.3) (layers "F.Cu" "B.Cu") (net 30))
 (segment (start 158 101.624999) (end 146.624999 101.624999) (width 0.2) (layer "B.Cu") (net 30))
 (segment (start 143.23 98.23) (end 143.23 92.305) (width 0.2) (layer "B.Cu") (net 30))
 (segment (start 146.624999 101.624999) (end 143.23 98.23) (width 0.2) (layer "B.Cu") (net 30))
 (segment (start 161.326001 100.673999) (end 161.399 100.601) (width 0.2) (layer "F.Cu") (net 26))
 (segment (start 161.399 100.5) (end 161.399 90.498) (width 0.2) (layer "F.Cu") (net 26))
 (segment (start 161.399 100.601) (end 161.399 100.5) (width 0.2) (layer "F.Cu") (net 26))
 (segment (start 161.251 100.673999) (end 161.326001 100.673999) (width 0.2) (layer "F.Cu") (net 26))
 (segment (start 161.399 90.498) (end 159.401 88.5) (width 0.2) (layer "F.Cu") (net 26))
 (segment (start 160.949999 100.975) (end 161.251 100.673999) (width 0.2) (layer "F.Cu") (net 26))
 (segment (start 161.399 100.5) (end 161.399 99) (width 0.2) (layer "F.Cu") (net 26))
 (segment (start 160 100.975) (end 160.949999 100.975) (width 0.2) (layer "F.Cu") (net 26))
 (segment (start 158.075 102.925) (end 160 102.925) (width 0.2) (layer "F.Cu") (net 28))
 (segment (start 158 103) (end 158.075 102.925) (width 0.2) (layer "F.Cu") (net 28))
 (via (at 158 103) (size 0.6) (drill 0.3) (layers "F.Cu" "B.Cu") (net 28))
 (segment (start 145.5 103) (end 138.15 95.65) (width 0.2) (layer "B.Cu") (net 28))
 (segment (start 158 103) (end 145.5 103) (width 0.2) (layer "B.Cu") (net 28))
 (segment (start 138.15 95.65) (end 138.15 92.305) (width 0.2) (layer "B.Cu") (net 28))
 (segment (start 156.5 101.00513) (end 156.5 106.14) (width 0.2) (layer "F.Cu") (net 10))
 (segment (start 153 98.375) (end 153.86987 98.375) (width 0.2) (layer "F.Cu") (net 10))
 (segment (start 156.5 106.14) (end 158.74 108.38) (width 0.2) (layer "F.Cu") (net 10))
 (segment (start 153.86987 98.375) (end 156.5 101.00513) (width 0.2) (layer "F.Cu") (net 10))
 (segment (start 154.748943 101.20266) (end 155.101 101.554717) (width 0.2) (layer "F.Cu") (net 13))
 (segment (start 155.101 101.554717) (end 155.101 102.40466) (width 0.2) (layer "F.Cu") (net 13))
 (segment (start 153 100.325) (end 153.86987 100.325) (width 0.2) (layer "F.Cu") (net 13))
 (segment (start 155.101 104.399) (end 151.12 108.38) (width 0.2) (layer "F.Cu") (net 13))
 (segment (start 155.101 102.40466) (end 155.101 104.399) (width 0.2) (layer "F.Cu") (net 13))
 (segment (start 153.86987 100.325) (end 154.74753 101.20266) (width 0.2) (layer "F.Cu") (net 13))
 (segment (start 154.74753 101.20266) (end 154.748943 101.20266) (width 0.2) (layer "F.Cu") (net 13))
 (segment (start 151.401 103.68516) (end 151.401 101.624001) (width 0.2) (layer "F.Cu") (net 37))
 (segment (start 151.401 101.624001) (end 152.050001 100.975) (width 0.2) (layer "F.Cu") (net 37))
 (segment (start 152.050001 100.975) (end 153 100.975) (width 0.2) (layer "F.Cu") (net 37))
 (segment (start 153.86987 100.975) (end 153 100.975) (width 0.2) (layer "F.Cu") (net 37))
 (segment (start 139 106.5) (end 148.58616 106.5) (width 0.2) (layer "F.Cu") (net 37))
 (segment (start 148.58616 106.5) (end 151.401 103.68516) (width 0.2) (layer "F.Cu") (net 37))
 (via (at 139 106.5) (size 0.6) (drill 0.3) (layers "F.Cu" "B.Cu") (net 37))
 (segment (start 136.10104 113) (end 135.5 113) (width 0.2) (layer "B.Cu") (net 37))
 (segment (start 139 110.10104) (end 136.10104 113) (width 0.2) (layer "B.Cu") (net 37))
 (segment (start 139 106.5) (end 139 110.10104) (width 0.2) (layer "B.Cu") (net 37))
 (segment (start 158.575 103.575) (end 160 103.575) (width 0.2) (layer "F.Cu") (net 27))
 (segment (start 158.575 103.6) (end 158.575 103.575) (width 0.2) (layer "F.Cu") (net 27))
 (segment (start 157.1 103.6) (end 158.575 103.6) (width 0.2) (layer "F.Cu") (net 27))
 (via (at 157.1 103.6) (size 0.6) (drill 0.3) (layers "F.Cu" "B.Cu") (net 27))
 (segment (start 144.1 103.6) (end 135.61 95.11) (width 0.2) (layer "B.Cu") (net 27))
 (segment (start 135.61 95.11) (end 135.61 92.305) (width 0.2) (layer "B.Cu") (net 27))
 (segment (start 157.1 103.6) (end 144.1 103.6) (width 0.2) (layer "B.Cu") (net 27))
 (segment (start 155.502 106.538) (end 153.66 108.38) (width 0.2) (layer "F.Cu") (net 12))
 (segment (start 153.949999 99.675) (end 155.502 101.227001) (width 0.2) (layer "F.Cu") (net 12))
 (segment (start 153 99.675) (end 153.949999 99.675) (width 0.2) (layer "F.Cu") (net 12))
 (segment (start 155.502 101.227001) (end 155.502 106.538) (width 0.2) (layer "F.Cu") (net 12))
 (segment (start 157.309313 102.275) (end 160 102.275) (width 0.2) (layer "F.Cu") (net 29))
 (via (at 157.309313 102.275) (size 0.6) (drill 0.3) (layers "F.Cu" "B.Cu") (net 29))
 (segment (start 157.309313 102.275) (end 146.275 102.275) (width 0.2) (layer "B.Cu") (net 29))
 (segment (start 146.275 102.275) (end 140.69 96.69) (width 0.2) (layer "B.Cu") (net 29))
 (segment (start 140.69 96.69) (end 140.69 92.305) (width 0.2) (layer "B.Cu") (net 29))
 (segment (start 155.5 100.575001) (end 155.502771 100.575001) (width 0.2) (layer "F.Cu") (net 11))
 (segment (start 155.502771 100.575001) (end 156 101.07223) (width 0.2) (layer "F.Cu") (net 11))
 (segment (start 156 101.07223) (end 156 108.18) (width 0.2) (layer "F.Cu") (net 11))
 (segment (start 153.949999 99.025) (end 155.5 100.575001) (width 0.2) (layer "F.Cu") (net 11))
 (segment (start 156 108.18) (end 156.2 108.38) (width 0.2) (layer "F.Cu") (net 11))
 (segment (start 153 99.025) (end 153.949999 99.025) (width 0.2) (layer "F.Cu") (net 11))
 (segment (start 156.5 96.5) (end 157.075 97.075) (width 0.2) (layer "F.Cu") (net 24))
 (segment (start 157.075 97.075) (end 160 97.075) (width 0.2) (layer "F.Cu") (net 24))
 (via (at 156.5 96.5) (size 0.6) (drill 0.3) (layers "F.Cu" "B.Cu") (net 24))
 (segment (start 160.998 116.002) (end 154.5 122.5) (width 0.2) (layer "B.Cu") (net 24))
 (segment (start 160.998 101.7641) (end 160.998 116.002) (width 0.2) (layer "B.Cu") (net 24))
 (segment (start 155 82.5) (end 156.9 84.4) (width 0.2) (layer "B.Cu") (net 24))
 (segment (start 156.9 84.4) (end 156.9 97.6661) (width 0.2) (layer "B.Cu") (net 24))
 (segment (start 144 82.5) (end 155 82.5) (width 0.2) (layer "B.Cu") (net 24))
 (segment (start 139.5 78) (end 144 82.5) (width 0.2) (layer "B.Cu") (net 24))
 (segment (start 156.9 97.6661) (end 160.998 101.7641) (width 0.2) (layer "B.Cu") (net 24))
 (segment (start 158.5 97.725) (end 160 97.725) (width 0.2) (layer "F.Cu") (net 25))
 (via (at 158.5 97.725) (size 0.6) (drill 0.3) (layers "F.Cu" "B.Cu") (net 25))
 (segment (start 157.34853 97.5) (end 157.301 97.5) (width 0.2) (layer "B.Cu") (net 25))
 (segment (start 155 125) (end 152.5 122.5) (width 0.2) (layer "B.Cu") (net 25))
 (segment (start 141.5 78) (end 145 81.5) (width 0.2) (layer "B.Cu") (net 25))
 (segment (start 161.399 122.101) (end 158.5 125) (width 0.2) (layer "B.Cu") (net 25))
 (segment (start 155.5 81.5) (end 157.301 83.301) (width 0.2) (layer "B.Cu") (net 25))
 (segment (start 158.5 125) (end 155 125) (width 0.2) (layer "B.Cu") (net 25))
 (segment (start 161.399 101.598) (end 161.399 122.101) (width 0.2) (layer "B.Cu") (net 25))
 (segment (start 157.301 97.5) (end 161.399 101.598) (width 0.2) (layer "B.Cu") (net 25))
 (segment (start 157.301 83.301) (end 157.301 97.5) (width 0.2) (layer "B.Cu") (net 25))
 (segment (start 145 81.5) (end 155.5 81.5) (width 0.2) (layer "B.Cu") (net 25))
 (segment (start 157.57353 97.725) (end 157.34853 97.5) (width 0.2) (layer "B.Cu") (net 25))
 (segment (start 158.5 97.725) (end 157.57353 97.725) (width 0.2) (layer "B.Cu") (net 25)))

